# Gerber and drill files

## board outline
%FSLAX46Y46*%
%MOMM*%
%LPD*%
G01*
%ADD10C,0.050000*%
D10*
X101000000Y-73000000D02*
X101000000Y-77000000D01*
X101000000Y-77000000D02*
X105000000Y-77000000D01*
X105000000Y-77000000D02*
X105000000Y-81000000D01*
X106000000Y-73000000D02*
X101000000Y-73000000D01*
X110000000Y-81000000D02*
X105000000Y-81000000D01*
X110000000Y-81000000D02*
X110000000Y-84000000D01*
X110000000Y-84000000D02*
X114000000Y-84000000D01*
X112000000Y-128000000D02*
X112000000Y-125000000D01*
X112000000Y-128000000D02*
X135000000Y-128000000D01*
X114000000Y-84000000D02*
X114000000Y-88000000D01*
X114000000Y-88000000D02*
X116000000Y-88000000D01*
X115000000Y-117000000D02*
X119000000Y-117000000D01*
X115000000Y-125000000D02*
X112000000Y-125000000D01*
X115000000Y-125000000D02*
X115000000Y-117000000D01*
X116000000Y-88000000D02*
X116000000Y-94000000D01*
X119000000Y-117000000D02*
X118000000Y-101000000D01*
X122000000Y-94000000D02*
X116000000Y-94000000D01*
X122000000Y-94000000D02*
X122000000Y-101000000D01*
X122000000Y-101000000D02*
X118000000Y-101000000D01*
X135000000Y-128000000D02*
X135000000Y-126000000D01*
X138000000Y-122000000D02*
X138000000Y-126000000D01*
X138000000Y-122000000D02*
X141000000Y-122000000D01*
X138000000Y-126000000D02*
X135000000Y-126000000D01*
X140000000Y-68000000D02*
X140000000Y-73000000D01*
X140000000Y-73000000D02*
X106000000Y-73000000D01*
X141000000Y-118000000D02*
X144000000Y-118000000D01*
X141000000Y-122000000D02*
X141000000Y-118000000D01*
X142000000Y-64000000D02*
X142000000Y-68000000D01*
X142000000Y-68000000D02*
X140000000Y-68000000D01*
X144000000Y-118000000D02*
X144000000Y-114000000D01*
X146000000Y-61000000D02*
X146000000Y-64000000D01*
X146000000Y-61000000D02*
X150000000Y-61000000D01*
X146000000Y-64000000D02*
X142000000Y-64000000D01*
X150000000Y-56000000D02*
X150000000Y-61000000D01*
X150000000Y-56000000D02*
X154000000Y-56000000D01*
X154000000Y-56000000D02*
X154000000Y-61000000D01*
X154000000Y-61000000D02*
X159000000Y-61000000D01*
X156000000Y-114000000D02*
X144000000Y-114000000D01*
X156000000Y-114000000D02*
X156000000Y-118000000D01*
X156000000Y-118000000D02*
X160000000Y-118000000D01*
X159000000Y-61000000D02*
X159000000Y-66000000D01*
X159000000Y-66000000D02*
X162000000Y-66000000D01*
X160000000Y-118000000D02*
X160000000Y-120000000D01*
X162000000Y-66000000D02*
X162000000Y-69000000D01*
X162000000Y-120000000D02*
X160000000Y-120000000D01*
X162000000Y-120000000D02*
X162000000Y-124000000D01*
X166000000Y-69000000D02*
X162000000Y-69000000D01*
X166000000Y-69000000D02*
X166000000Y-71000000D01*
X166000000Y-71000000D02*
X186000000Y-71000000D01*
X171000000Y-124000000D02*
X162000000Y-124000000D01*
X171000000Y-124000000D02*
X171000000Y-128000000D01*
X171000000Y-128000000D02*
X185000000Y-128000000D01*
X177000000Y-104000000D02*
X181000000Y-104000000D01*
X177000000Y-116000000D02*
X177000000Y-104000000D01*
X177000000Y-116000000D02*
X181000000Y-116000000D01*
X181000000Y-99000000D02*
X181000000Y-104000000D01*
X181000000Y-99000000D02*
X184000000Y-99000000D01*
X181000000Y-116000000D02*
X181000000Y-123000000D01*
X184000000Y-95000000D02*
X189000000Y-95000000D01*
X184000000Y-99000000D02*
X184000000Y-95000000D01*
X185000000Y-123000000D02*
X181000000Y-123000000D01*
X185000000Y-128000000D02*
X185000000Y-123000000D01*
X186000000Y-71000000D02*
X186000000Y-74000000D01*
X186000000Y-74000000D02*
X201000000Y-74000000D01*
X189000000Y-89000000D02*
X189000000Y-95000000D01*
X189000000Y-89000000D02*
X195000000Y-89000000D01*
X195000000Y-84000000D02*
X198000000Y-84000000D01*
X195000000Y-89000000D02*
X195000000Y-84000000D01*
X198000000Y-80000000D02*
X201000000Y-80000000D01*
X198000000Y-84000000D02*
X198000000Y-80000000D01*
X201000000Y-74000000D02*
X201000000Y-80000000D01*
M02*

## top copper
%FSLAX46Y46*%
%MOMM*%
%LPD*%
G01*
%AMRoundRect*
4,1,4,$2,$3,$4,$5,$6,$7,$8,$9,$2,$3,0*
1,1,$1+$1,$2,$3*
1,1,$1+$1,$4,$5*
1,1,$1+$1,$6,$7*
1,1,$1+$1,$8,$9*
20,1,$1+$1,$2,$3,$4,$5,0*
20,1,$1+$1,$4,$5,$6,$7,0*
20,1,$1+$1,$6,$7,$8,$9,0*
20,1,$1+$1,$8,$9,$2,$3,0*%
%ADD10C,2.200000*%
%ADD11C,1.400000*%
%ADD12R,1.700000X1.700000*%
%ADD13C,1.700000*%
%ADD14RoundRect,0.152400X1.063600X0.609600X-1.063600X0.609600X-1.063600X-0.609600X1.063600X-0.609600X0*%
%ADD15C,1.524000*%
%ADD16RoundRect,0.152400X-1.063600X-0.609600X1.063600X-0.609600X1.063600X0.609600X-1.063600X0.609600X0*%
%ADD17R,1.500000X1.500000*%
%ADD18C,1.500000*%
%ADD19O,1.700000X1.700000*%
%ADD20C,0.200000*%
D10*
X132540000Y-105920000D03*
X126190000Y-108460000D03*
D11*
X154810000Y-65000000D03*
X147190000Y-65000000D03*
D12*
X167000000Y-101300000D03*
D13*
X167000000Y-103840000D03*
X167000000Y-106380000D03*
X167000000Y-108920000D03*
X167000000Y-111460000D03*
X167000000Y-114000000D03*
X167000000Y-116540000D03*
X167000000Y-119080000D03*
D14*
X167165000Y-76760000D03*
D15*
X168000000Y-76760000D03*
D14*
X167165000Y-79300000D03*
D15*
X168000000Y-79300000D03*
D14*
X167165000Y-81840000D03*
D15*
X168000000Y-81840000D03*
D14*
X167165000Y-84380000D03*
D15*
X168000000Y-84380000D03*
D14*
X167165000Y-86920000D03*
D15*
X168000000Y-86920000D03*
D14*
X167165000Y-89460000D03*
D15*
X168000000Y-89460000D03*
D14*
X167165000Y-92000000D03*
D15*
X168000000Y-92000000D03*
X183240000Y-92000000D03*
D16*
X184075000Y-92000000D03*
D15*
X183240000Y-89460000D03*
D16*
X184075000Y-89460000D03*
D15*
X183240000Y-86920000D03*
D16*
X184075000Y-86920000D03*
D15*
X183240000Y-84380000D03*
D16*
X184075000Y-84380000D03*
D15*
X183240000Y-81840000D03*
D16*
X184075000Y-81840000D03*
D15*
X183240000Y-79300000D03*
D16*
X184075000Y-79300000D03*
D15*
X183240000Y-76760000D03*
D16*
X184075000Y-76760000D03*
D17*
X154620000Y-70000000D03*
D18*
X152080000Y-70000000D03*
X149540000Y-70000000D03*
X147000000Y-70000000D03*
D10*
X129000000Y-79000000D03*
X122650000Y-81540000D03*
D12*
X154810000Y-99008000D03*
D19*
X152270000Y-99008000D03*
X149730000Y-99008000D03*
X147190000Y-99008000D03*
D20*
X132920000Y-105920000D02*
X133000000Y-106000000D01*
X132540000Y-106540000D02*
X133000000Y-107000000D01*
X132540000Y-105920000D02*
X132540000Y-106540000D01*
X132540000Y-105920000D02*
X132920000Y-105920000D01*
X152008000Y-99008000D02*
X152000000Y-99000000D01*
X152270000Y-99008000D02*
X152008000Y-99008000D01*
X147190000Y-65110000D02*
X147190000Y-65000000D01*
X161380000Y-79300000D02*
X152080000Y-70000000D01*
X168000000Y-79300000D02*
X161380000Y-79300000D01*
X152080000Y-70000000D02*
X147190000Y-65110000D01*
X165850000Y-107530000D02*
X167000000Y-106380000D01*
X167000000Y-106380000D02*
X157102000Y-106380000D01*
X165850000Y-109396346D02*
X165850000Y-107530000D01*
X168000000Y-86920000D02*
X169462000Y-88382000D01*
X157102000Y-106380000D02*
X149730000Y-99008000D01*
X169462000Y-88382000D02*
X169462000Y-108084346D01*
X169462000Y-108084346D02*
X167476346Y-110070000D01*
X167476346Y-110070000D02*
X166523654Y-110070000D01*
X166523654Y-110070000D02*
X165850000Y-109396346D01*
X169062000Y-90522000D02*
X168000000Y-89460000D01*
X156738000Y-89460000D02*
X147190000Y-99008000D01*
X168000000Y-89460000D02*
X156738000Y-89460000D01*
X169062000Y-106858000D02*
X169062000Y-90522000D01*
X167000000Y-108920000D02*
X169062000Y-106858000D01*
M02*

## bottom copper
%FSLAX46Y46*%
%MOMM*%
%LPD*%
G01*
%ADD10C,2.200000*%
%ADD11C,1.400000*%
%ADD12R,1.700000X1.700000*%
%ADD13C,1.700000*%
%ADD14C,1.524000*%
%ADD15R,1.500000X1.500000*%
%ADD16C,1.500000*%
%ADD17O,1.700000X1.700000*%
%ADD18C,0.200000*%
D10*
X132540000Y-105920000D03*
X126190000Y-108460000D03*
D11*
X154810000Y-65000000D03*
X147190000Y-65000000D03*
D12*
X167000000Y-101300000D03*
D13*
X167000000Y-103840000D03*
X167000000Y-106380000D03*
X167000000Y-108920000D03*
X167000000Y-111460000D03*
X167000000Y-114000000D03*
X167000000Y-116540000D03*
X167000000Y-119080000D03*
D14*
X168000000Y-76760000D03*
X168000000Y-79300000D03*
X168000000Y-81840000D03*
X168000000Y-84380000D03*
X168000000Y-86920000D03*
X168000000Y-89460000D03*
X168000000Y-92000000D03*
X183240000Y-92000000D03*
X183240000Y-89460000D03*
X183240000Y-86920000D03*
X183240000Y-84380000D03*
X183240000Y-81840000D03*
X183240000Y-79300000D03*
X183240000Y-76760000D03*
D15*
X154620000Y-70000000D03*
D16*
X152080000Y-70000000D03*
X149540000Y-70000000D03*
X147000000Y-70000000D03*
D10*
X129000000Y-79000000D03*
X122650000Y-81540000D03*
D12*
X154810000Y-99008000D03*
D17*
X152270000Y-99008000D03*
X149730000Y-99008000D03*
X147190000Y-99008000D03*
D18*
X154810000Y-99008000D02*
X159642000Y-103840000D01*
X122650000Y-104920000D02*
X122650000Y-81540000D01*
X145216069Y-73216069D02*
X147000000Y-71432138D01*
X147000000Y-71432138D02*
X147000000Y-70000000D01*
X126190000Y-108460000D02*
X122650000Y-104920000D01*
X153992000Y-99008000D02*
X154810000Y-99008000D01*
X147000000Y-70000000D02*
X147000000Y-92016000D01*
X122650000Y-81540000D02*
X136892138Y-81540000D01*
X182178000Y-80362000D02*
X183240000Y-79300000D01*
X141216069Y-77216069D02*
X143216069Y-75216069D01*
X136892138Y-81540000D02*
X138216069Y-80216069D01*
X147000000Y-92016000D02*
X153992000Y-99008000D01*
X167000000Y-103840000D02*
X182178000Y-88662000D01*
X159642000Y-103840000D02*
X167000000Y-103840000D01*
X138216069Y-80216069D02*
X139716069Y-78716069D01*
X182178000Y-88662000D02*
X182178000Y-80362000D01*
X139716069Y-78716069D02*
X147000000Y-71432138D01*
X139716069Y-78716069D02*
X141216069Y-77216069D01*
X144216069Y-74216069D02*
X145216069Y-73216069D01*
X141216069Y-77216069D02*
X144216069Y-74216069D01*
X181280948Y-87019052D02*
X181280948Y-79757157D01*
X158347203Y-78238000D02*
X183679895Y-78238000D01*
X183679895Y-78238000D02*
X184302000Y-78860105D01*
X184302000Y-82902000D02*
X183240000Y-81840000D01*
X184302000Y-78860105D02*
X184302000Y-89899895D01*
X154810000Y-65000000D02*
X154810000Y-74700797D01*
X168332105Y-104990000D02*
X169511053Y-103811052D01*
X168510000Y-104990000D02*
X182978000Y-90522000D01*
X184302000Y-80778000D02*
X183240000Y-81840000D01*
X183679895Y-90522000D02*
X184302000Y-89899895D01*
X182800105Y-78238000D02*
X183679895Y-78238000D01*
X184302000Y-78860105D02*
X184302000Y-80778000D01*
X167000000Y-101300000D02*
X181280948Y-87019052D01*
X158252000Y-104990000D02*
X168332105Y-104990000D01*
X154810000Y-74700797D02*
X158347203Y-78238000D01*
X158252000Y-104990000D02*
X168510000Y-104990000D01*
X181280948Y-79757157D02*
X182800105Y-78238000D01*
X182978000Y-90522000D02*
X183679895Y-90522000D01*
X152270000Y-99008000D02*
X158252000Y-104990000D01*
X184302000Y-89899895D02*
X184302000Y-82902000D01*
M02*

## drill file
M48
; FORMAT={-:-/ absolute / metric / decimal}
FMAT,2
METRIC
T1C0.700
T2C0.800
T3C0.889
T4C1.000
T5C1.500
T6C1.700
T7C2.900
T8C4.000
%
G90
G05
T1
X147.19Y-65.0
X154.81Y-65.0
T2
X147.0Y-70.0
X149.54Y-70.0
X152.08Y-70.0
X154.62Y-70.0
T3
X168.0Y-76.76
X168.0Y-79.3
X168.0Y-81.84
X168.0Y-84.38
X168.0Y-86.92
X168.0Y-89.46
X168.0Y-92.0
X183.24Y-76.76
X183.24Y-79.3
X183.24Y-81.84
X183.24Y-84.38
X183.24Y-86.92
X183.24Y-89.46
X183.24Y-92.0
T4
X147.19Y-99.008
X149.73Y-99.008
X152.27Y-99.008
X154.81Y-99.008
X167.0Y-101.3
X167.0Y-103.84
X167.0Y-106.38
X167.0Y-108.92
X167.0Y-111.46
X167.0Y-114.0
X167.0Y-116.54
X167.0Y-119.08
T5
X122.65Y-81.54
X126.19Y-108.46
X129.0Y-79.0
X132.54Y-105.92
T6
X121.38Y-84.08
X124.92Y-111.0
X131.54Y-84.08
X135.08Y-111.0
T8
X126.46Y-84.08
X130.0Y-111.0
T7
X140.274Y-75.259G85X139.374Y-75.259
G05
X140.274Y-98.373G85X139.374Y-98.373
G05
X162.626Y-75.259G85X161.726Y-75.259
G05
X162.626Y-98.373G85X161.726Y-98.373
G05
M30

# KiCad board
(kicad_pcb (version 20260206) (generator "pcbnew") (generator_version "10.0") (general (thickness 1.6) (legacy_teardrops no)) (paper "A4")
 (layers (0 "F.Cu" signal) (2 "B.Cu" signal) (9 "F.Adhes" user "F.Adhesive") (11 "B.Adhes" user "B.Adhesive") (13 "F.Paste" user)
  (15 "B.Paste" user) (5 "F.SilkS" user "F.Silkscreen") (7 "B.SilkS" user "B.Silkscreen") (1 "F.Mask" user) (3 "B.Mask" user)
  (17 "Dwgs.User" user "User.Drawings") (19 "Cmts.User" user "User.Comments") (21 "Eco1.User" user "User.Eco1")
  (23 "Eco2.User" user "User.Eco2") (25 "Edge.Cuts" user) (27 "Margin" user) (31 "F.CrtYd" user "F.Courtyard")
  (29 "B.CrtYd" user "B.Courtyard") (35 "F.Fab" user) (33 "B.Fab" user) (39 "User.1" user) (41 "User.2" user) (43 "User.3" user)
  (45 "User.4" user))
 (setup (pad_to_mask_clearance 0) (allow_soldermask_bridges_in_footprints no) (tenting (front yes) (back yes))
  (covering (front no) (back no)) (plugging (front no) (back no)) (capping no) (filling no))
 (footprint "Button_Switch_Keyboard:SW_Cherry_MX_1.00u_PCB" (layer "F.Cu") (at 132.54 105.92)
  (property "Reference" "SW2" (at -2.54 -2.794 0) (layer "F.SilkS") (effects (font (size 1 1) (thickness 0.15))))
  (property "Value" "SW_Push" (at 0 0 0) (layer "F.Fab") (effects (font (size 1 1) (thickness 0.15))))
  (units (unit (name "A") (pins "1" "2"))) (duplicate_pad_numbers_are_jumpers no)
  (pad "" np_thru_hole circle (at -7.62 5.08) (size 1.7 1.7) (drill 1.7) (layers "*.Cu" "*.Mask"))
  (pad "" np_thru_hole circle (at -2.54 5.08) (size 4 4) (drill 4) (layers "*.Cu" "*.Mask"))
  (pad "" np_thru_hole circle (at 2.54 5.08) (size 1.7 1.7) (drill 1.7) (layers "*.Cu" "*.Mask"))
  (pad "1" thru_hole circle (at 0 0) (size 2.2 2.2) (drill 1.5) (layers "*.Cu" "*.Mask") (remove_unused_layers no) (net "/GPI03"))
  (pad "2" thru_hole circle (at -6.35 2.54) (size 2.2 2.2) (drill 1.5) (layers "*.Cu" "*.Mask") (remove_unused_layers no) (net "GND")))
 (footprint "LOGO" (layer "F.Cu") (at 160 112)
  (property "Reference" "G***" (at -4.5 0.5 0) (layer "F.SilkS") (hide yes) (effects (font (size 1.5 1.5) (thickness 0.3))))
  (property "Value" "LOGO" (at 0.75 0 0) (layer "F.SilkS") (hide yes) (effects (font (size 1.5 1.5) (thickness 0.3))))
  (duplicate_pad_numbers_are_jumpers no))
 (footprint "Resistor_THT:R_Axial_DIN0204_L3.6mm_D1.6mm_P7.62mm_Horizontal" (layer "F.Cu") (at 154.81 65 180)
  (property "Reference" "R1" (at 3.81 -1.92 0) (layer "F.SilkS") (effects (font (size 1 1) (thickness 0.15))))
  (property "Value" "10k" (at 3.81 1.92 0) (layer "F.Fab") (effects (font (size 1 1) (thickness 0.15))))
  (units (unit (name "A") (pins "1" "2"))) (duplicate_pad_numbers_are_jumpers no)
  (pad "1" thru_hole circle (at 0 0 180) (size 1.4 1.4) (drill 0.7) (layers "*.Cu" "*.Mask") (remove_unused_layers no) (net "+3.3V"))
  (pad "2" thru_hole circle (at 7.62 0 180) (size 1.4 1.4) (drill 0.7) (layers "*.Cu" "*.Mask") (remove_unused_layers no)
   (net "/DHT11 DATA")))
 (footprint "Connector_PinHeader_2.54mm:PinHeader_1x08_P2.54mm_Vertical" (layer "F.Cu") (at 167 101.3)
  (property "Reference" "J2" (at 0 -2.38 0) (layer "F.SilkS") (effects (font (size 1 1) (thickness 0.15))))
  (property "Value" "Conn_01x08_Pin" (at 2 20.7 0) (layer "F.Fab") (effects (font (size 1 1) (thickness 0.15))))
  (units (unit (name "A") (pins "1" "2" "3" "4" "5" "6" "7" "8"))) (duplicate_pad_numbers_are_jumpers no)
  (pad "1" thru_hole rect (at 0 0) (size 1.7 1.7) (drill 1) (layers "*.Cu" "*.Mask") (remove_unused_layers no) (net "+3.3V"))
  (pad "2" thru_hole circle (at 0 2.54) (size 1.7 1.7) (drill 1) (layers "*.Cu" "*.Mask") (remove_unused_layers no) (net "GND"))
  (pad "3" thru_hole circle (at 0 5.08) (size 1.7 1.7) (drill 1) (layers "*.Cu" "*.Mask") (remove_unused_layers no) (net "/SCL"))
  (pad "4" thru_hole circle (at 0 7.62) (size 1.7 1.7) (drill 1) (layers "*.Cu" "*.Mask") (remove_unused_layers no) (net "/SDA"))
  (pad "5" thru_hole circle (at 0 10.16) (size 1.7 1.7) (drill 1) (layers "*.Cu" "*.Mask") (remove_unused_layers no)
   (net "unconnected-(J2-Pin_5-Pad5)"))
  (pad "6" thru_hole circle (at 0 12.7) (size 1.7 1.7) (drill 1) (layers "*.Cu" "*.Mask") (remove_unused_layers no)
   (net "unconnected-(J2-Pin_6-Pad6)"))
  (pad "7" thru_hole circle (at 0 15.24) (size 1.7 1.7) (drill 1) (layers "*.Cu" "*.Mask") (remove_unused_layers no)
   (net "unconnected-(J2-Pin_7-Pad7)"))
  (pad "8" thru_hole circle (at 0 17.78) (size 1.7 1.7) (drill 1) (layers "*.Cu" "*.Mask") (remove_unused_layers no)
   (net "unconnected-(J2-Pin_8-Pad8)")))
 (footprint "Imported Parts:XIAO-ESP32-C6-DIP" (layer "F.Cu") (at 175.62 84.38 90)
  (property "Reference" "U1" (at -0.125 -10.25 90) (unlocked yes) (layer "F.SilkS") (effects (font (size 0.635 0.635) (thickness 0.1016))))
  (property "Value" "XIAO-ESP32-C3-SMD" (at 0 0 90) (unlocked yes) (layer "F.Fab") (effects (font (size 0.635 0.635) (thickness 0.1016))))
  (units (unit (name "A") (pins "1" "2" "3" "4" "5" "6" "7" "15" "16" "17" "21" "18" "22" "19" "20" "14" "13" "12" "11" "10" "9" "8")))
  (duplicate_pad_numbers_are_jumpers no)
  (pad "1" smd roundrect (at 7.62 -8.455 180) (size 2.432 1.524) (layers "F.Cu" "F.Mask") (roundrect_rratio 0.1)
   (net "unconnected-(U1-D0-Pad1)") (thermal_bridge_angle 45))
  (pad "1" thru_hole circle (at 7.62 -7.62 180) (size 1.524 1.524) (drill 0.889) (layers "*.Cu" "*.Mask") (remove_unused_layers no)
   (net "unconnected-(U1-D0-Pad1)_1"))
  (pad "2" smd roundrect (at 5.08 -8.455 180) (size 2.432 1.524) (layers "F.Cu" "F.Mask") (roundrect_rratio 0.1) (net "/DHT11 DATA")
   (thermal_bridge_angle 45))
  (pad "2" thru_hole circle (at 5.08 -7.62 180) (size 1.524 1.524) (drill 0.889) (layers "*.Cu" "*.Mask") (remove_unused_layers no)
   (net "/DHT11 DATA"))
  (pad "3" smd roundrect (at 2.54 -8.455 180) (size 2.432 1.524) (layers "F.Cu" "F.Mask") (roundrect_rratio 0.1) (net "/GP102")
   (thermal_bridge_angle 45))
  (pad "3" thru_hole circle (at 2.54 -7.62 180) (size 1.524 1.524) (drill 0.889) (layers "*.Cu" "*.Mask") (remove_unused_layers no)
   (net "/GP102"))
  (pad "4" smd roundrect (at 0 -8.455 180) (size 2.432 1.524) (layers "F.Cu" "F.Mask") (roundrect_rratio 0.1) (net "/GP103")
   (thermal_bridge_angle 45))
  (pad "4" thru_hole circle (at 0 -7.62 180) (size 1.524 1.524) (drill 0.889) (layers "*.Cu" "*.Mask") (remove_unused_layers no)
   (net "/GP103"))
  (pad "5" smd roundrect (at -2.54 -8.455 180) (size 2.432 1.524) (layers "F.Cu" "F.Mask") (roundrect_rratio 0.1) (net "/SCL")
   (thermal_bridge_angle 45))
  (pad "5" thru_hole circle (at -2.54 -7.62 180) (size 1.524 1.524) (drill 0.889) (layers "*.Cu" "*.Mask") (remove_unused_layers no)
   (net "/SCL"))
  (pad "6" smd roundrect (at -5.08 -8.455 180) (size 2.432 1.524) (layers "F.Cu" "F.Mask") (roundrect_rratio 0.1) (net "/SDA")
   (thermal_bridge_angle 45))
  (pad "6" thru_hole circle (at -5.08 -7.62 180) (size 1.524 1.524) (drill 0.889) (layers "*.Cu" "*.Mask") (remove_unused_layers no)
   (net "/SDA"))
  (pad "7" smd roundrect (at -7.62 -8.455 180) (size 2.432 1.524) (layers "F.Cu" "F.Mask") (roundrect_rratio 0.1)
   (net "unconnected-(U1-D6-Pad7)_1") (thermal_bridge_angle 45))
  (pad "7" thru_hole circle (at -7.62 -7.62 180) (size 1.524 1.524) (drill 0.889) (layers "*.Cu" "*.Mask") (remove_unused_layers no)
   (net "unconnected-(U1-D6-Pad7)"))
  (pad "8" thru_hole circle (at -7.62 7.62) (size 1.524 1.524) (drill 0.889) (layers "*.Cu" "*.Mask") (remove_unused_layers no)
   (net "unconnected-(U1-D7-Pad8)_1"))
  (pad "8" smd roundrect (at -7.62 8.455) (size 2.432 1.524) (layers "F.Cu" "F.Mask") (roundrect_rratio 0.1)
   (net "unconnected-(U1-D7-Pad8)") (thermal_bridge_angle 45))
  (pad "9" thru_hole circle (at -5.08 7.62) (size 1.524 1.524) (drill 0.889) (layers "*.Cu" "*.Mask") (remove_unused_layers no)
   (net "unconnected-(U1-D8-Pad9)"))
  (pad "9" smd roundrect (at -5.08 8.455) (size 2.432 1.524) (layers "F.Cu" "F.Mask") (roundrect_rratio 0.1)
   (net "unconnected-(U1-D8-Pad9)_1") (thermal_bridge_angle 45))
  (pad "10" thru_hole circle (at -2.54 7.62) (size 1.524 1.524) (drill 0.889) (layers "*.Cu" "*.Mask") (remove_unused_layers no)
   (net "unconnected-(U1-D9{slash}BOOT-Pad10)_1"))
  (pad "10" smd roundrect (at -2.54 8.455) (size 2.432 1.524) (layers "F.Cu" "F.Mask") (roundrect_rratio 0.1)
   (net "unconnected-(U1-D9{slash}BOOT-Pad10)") (thermal_bridge_angle 45))
  (pad "11" thru_hole circle (at 0 7.62) (size 1.524 1.524) (drill 0.889) (layers "*.Cu" "*.Mask") (remove_unused_layers no)
   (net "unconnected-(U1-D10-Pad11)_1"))
  (pad "11" smd roundrect (at 0 8.455) (size 2.432 1.524) (layers "F.Cu" "F.Mask") (roundrect_rratio 0.1) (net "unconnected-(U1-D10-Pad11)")
   (thermal_bridge_angle 45))
  (pad "12" thru_hole circle (at 2.54 7.62) (size 1.524 1.524) (drill 0.889) (layers "*.Cu" "*.Mask") (remove_unused_layers no)
   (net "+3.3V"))
  (pad "12" smd roundrect (at 2.54 8.455) (size 2.432 1.524) (layers "F.Cu" "F.Mask") (roundrect_rratio 0.1) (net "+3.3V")
   (thermal_bridge_angle 45))
  (pad "13" thru_hole circle (at 5.08 7.62) (size 1.524 1.524) (drill 0.889) (layers "*.Cu" "*.Mask") (remove_unused_layers no) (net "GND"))
  (pad "13" smd roundrect (at 5.08 8.455) (size 2.432 1.524) (layers "F.Cu" "F.Mask") (roundrect_rratio 0.1) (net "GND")
   (thermal_bridge_angle 45))
  (pad "14" thru_hole circle (at 7.62 7.62) (size 1.524 1.524) (drill 0.889) (layers "*.Cu" "*.Mask") (remove_unused_layers no) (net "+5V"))
  (pad "14" smd roundrect (at 7.62 8.455) (size 2.432 1.524) (layers "F.Cu" "F.Mask") (roundrect_rratio 0.1) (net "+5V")
   (thermal_bridge_angle 45)))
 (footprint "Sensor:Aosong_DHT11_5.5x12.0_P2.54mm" (layer "F.Cu") (at 154.62 70 -90)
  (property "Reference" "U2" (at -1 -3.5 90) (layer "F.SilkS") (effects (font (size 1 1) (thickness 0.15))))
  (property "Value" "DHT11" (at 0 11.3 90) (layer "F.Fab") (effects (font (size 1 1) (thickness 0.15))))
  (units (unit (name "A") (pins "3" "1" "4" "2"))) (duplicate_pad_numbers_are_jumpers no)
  (pad "1" thru_hole rect (at 0 0 270) (size 1.5 1.5) (drill 0.8) (layers "*.Cu" "*.Mask") (remove_unused_layers no) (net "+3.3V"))
  (pad "2" thru_hole circle (at 0 2.54 270) (size 1.5 1.5) (drill 0.8) (layers "*.Cu" "*.Mask") (remove_unused_layers no)
   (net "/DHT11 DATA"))
  (pad "3" thru_hole circle (at 0 5.08 270) (size 1.5 1.5) (drill 0.8) (layers "*.Cu" "*.Mask") (remove_unused_layers no)
   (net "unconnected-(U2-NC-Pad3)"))
  (pad "4" thru_hole circle (at 0 7.62 270) (size 1.5 1.5) (drill 0.8) (layers "*.Cu" "*.Mask") (remove_unused_layers no) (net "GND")))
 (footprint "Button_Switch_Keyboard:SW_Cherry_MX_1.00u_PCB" (layer "F.Cu") (at 129 79)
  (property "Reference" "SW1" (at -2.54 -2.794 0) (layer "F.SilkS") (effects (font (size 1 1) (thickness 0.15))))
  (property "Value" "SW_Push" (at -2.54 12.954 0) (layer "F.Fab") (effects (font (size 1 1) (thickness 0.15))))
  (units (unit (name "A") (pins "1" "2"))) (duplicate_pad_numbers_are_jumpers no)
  (pad "" np_thru_hole circle (at -7.62 5.08) (size 1.7 1.7) (drill 1.7) (layers "*.Cu" "*.Mask"))
  (pad "" np_thru_hole circle (at -2.54 5.08) (size 4 4) (drill 4) (layers "*.Cu" "*.Mask"))
  (pad "" np_thru_hole circle (at 2.54 5.08) (size 1.7 1.7) (drill 1.7) (layers "*.Cu" "*.Mask"))
  (pad "1" thru_hole circle (at 0 0) (size 2.2 2.2) (drill 1.5) (layers "*.Cu" "*.Mask") (remove_unused_layers no) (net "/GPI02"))
  (pad "2" thru_hole circle (at -6.35 2.54) (size 2.2 2.2) (drill 1.5) (layers "*.Cu" "*.Mask") (remove_unused_layers no) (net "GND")))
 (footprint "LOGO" (layer "F.Cu") (at 191.5 80.5)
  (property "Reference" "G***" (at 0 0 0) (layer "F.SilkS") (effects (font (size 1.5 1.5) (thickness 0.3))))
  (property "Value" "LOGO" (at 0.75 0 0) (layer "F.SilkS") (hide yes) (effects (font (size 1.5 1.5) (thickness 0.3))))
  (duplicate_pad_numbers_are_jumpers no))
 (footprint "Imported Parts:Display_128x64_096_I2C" (layer "F.Cu") (at 151 99.008 180)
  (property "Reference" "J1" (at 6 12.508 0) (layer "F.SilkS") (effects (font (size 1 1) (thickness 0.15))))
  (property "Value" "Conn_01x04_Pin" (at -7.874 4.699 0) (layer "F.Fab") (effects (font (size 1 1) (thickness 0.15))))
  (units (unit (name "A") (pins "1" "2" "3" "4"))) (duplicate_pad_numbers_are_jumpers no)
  (pad "" np_thru_hole oval (at -11.176 0.635 180) (size 3.8 2.9) (drill oval 3.8 2.9) (layers "*.Cu" "*.Mask"))
  (pad "" np_thru_hole oval (at -11.176 23.749 180) (size 3.8 2.9) (drill oval 3.8 2.9) (layers "*.Cu" "*.Mask"))
  (pad "" np_thru_hole oval (at 11.176 0.635 180) (size 3.8 2.9) (drill oval 3.8 2.9) (layers "*.Cu" "*.Mask"))
  (pad "" np_thru_hole oval (at 11.176 23.749 180) (size 3.8 2.9) (drill oval 3.8 2.9) (layers "*.Cu" "*.Mask"))
  (pad "1" thru_hole rect (at -3.81 0 270) (size 1.7 1.7) (drill 1) (layers "*.Cu" "*.Mask") (remove_unused_layers no) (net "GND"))
  (pad "2" thru_hole oval (at -1.27 0 270) (size 1.7 1.7) (drill 1) (layers "*.Cu" "*.Mask") (remove_unused_layers no) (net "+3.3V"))
  (pad "3" thru_hole oval (at 1.27 0 270) (size 1.7 1.7) (drill 1) (layers "*.Cu" "*.Mask") (remove_unused_layers no) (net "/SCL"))
  (pad "4" thru_hole oval (at 3.81 0 270) (size 1.7 1.7) (drill 1) (layers "*.Cu" "*.Mask") (remove_unused_layers no) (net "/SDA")))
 (gr_line (start 101 73) (end 101 77) (stroke (width 0.05) (type default)) (layer "Edge.Cuts"))
 (gr_line (start 101 77) (end 105 77) (stroke (width 0.05) (type default)) (layer "Edge.Cuts"))
 (gr_line (start 105 77) (end 105 81) (stroke (width 0.05) (type default)) (layer "Edge.Cuts"))
 (gr_line (start 106 73) (end 101 73) (stroke (width 0.05) (type default)) (layer "Edge.Cuts"))
 (gr_line (start 110 81) (end 105 81) (stroke (width 0.05) (type default)) (layer "Edge.Cuts"))
 (gr_line (start 110 81) (end 110 84) (stroke (width 0.05) (type default)) (layer "Edge.Cuts"))
 (gr_line (start 110 84) (end 114 84) (stroke (width 0.05) (type default)) (layer "Edge.Cuts"))
 (gr_line (start 112 128) (end 112 125) (stroke (width 0.05) (type default)) (layer "Edge.Cuts"))
 (gr_line (start 112 128) (end 135 128) (stroke (width 0.05) (type default)) (layer "Edge.Cuts"))
 (gr_line (start 114 84) (end 114 88) (stroke (width 0.05) (type default)) (layer "Edge.Cuts"))
 (gr_line (start 114 88) (end 116 88) (stroke (width 0.05) (type default)) (layer "Edge.Cuts"))
 (gr_line (start 115 117) (end 119 117) (stroke (width 0.05) (type default)) (layer "Edge.Cuts"))
 (gr_line (start 115 125) (end 112 125) (stroke (width 0.05) (type default)) (layer "Edge.Cuts"))
 (gr_line (start 115 125) (end 115 117) (stroke (width 0.05) (type default)) (layer "Edge.Cuts"))
 (gr_line (start 116 88) (end 116 94) (stroke (width 0.05) (type default)) (layer "Edge.Cuts"))
 (gr_line (start 119 117) (end 118 101) (stroke (width 0.05) (type default)) (layer "Edge.Cuts"))
 (gr_line (start 122 94) (end 116 94) (stroke (width 0.05) (type default)) (layer "Edge.Cuts"))
 (gr_line (start 122 94) (end 122 101) (stroke (width 0.05) (type default)) (layer "Edge.Cuts"))
 (gr_line (start 122 101) (end 118 101) (stroke (width 0.05) (type default)) (layer "Edge.Cuts"))
 (gr_line (start 135 128) (end 135 126) (stroke (width 0.05) (type default)) (layer "Edge.Cuts"))
 (gr_line (start 138 122) (end 138 126) (stroke (width 0.05) (type default)) (layer "Edge.Cuts"))
 (gr_line (start 138 122) (end 141 122) (stroke (width 0.05) (type default)) (layer "Edge.Cuts"))
 (gr_line (start 138 126) (end 135 126) (stroke (width 0.05) (type default)) (layer "Edge.Cuts"))
 (gr_line (start 140 68) (end 140 73) (stroke (width 0.05) (type default)) (layer "Edge.Cuts"))
 (gr_line (start 140 73) (end 106 73) (stroke (width 0.05) (type default)) (layer "Edge.Cuts"))
 (gr_line (start 141 118) (end 144 118) (stroke (width 0.05) (type default)) (layer "Edge.Cuts"))
 (gr_line (start 141 122) (end 141 118) (stroke (width 0.05) (type default)) (layer "Edge.Cuts"))
 (gr_line (start 142 64) (end 142 68) (stroke (width 0.05) (type default)) (layer "Edge.Cuts"))
 (gr_line (start 142 68) (end 140 68) (stroke (width 0.05) (type default)) (layer "Edge.Cuts"))
 (gr_line (start 144 118) (end 144 114) (stroke (width 0.05) (type default)) (layer "Edge.Cuts"))
 (gr_line (start 146 61) (end 146 64) (stroke (width 0.05) (type default)) (layer "Edge.Cuts"))
 (gr_line (start 146 61) (end 150 61) (stroke (width 0.05) (type default)) (layer "Edge.Cuts"))
 (gr_line (start 146 64) (end 142 64) (stroke (width 0.05) (type default)) (layer "Edge.Cuts"))
 (gr_line (start 150 56) (end 150 61) (stroke (width 0.05) (type default)) (layer "Edge.Cuts"))
 (gr_line (start 150 56) (end 154 56) (stroke (width 0.05) (type default)) (layer "Edge.Cuts"))
 (gr_line (start 154 56) (end 154 61) (stroke (width 0.05) (type default)) (layer "Edge.Cuts"))
 (gr_line (start 154 61) (end 159 61) (stroke (width 0.05) (type default)) (layer "Edge.Cuts"))
 (gr_line (start 156 114) (end 144 114) (stroke (width 0.05) (type default)) (layer "Edge.Cuts"))
 (gr_line (start 156 114) (end 156 118) (stroke (width 0.05) (type default)) (layer "Edge.Cuts"))
 (gr_line (start 156 118) (end 160 118) (stroke (width 0.05) (type default)) (layer "Edge.Cuts"))
 (gr_line (start 159 61) (end 159 66) (stroke (width 0.05) (type default)) (layer "Edge.Cuts"))
 (gr_line (start 159 66) (end 162 66) (stroke (width 0.05) (type default)) (layer "Edge.Cuts"))
 (gr_line (start 160 118) (end 160 120) (stroke (width 0.05) (type default)) (layer "Edge.Cuts"))
 (gr_line (start 162 66) (end 162 69) (stroke (width 0.05) (type default)) (layer "Edge.Cuts"))
 (gr_line (start 162 120) (end 160 120) (stroke (width 0.05) (type default)) (layer "Edge.Cuts"))
 (gr_line (start 162 120) (end 162 124) (stroke (width 0.05) (type default)) (layer "Edge.Cuts"))
 (gr_line (start 166 69) (end 162 69) (stroke (width 0.05) (type default)) (layer "Edge.Cuts"))
 (gr_line (start 166 69) (end 166 71) (stroke (width 0.05) (type default)) (layer "Edge.Cuts"))
 (gr_line (start 166 71) (end 186 71) (stroke (width 0.05) (type default)) (layer "Edge.Cuts"))
 (gr_line (start 171 124) (end 162 124) (stroke (width 0.05) (type default)) (layer "Edge.Cuts"))
 (gr_line (start 171 124) (end 171 128) (stroke (width 0.05) (type default)) (layer "Edge.Cuts"))
 (gr_line (start 171 128) (end 185 128) (stroke (width 0.05) (type default)) (layer "Edge.Cuts"))
 (gr_line (start 177 104) (end 181 104) (stroke (width 0.05) (type default)) (layer "Edge.Cuts"))
 (gr_line (start 177 116) (end 177 104) (stroke (width 0.05) (type default)) (layer "Edge.Cuts"))
 (gr_line (start 177 116) (end 181 116) (stroke (width 0.05) (type default)) (layer "Edge.Cuts"))
 (gr_line (start 181 99) (end 181 104) (stroke (width 0.05) (type default)) (layer "Edge.Cuts"))
 (gr_line (start 181 99) (end 184 99) (stroke (width 0.05) (type default)) (layer "Edge.Cuts"))
 (gr_line (start 181 116) (end 181 123) (stroke (width 0.05) (type default)) (layer "Edge.Cuts"))
 (gr_line (start 184 95) (end 189 95) (stroke (width 0.05) (type default)) (layer "Edge.Cuts"))
 (gr_line (start 184 99) (end 184 95) (stroke (width 0.05) (type default)) (layer "Edge.Cuts"))
 (gr_line (start 185 123) (end 181 123) (stroke (width 0.05) (type default)) (layer "Edge.Cuts"))
 (gr_line (start 185 128) (end 185 123) (stroke (width 0.05) (type default)) (layer "Edge.Cuts"))
 (gr_line (start 186 71) (end 186 74) (stroke (width 0.05) (type default)) (layer "Edge.Cuts"))
 (gr_line (start 186 74) (end 201 74) (stroke (width 0.05) (type default)) (layer "Edge.Cuts"))
 (gr_line (start 189 89) (end 189 95) (stroke (width 0.05) (type default)) (layer "Edge.Cuts"))
 (gr_line (start 189 89) (end 195 89) (stroke (width 0.05) (type default)) (layer "Edge.Cuts"))
 (gr_line (start 195 84) (end 198 84) (stroke (width 0.05) (type default)) (layer "Edge.Cuts"))
 (gr_line (start 195 89) (end 195 84) (stroke (width 0.05) (type default)) (layer "Edge.Cuts"))
 (gr_line (start 198 80) (end 201 80) (stroke (width 0.05) (type default)) (layer "Edge.Cuts"))
 (gr_line (start 198 84) (end 198 80) (stroke (width 0.05) (type default)) (layer "Edge.Cuts"))
 (gr_line (start 201 74) (end 201 80) (stroke (width 0.05) (type default)) (layer "Edge.Cuts"))
 (segment (start 132.92 105.92) (end 133 106) (width 0.2) (layer "F.Cu") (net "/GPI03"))
 (segment (start 132.54 106.54) (end 133 107) (width 0.2) (layer "F.Cu") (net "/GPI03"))
 (segment (start 132.54 105.92) (end 132.54 106.54) (width 0.2) (layer "F.Cu") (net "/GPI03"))
 (segment (start 132.54 105.92) (end 132.92 105.92) (width 0.2) (layer "F.Cu") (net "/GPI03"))
 (segment (start 154.81 99.008) (end 159.642 103.84) (width 0.2) (layer "B.Cu") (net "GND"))
 (segment (start 122.65 104.92) (end 122.65 81.54) (width 0.2) (layer "B.Cu") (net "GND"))
 (segment (start 145.216069 73.216069) (end 147 71.432138) (width 0.2) (layer "B.Cu") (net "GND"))
 (segment (start 147 71.432138) (end 147 70) (width 0.2) (layer "B.Cu") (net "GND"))
 (segment (start 126.19 108.46) (end 122.65 104.92) (width 0.2) (layer "B.Cu") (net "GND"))
 (segment (start 153.992 99.008) (end 154.81 99.008) (width 0.2) (layer "B.Cu") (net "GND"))
 (segment (start 147 70) (end 147 92.016) (width 0.2) (layer "B.Cu") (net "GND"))
 (segment (start 122.65 81.54) (end 136.892138 81.54) (width 0.2) (layer "B.Cu") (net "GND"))
 (segment (start 182.178 80.362) (end 183.24 79.3) (width 0.2) (layer "B.Cu") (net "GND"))
 (segment (start 141.216069 77.216069) (end 143.216069 75.216069) (width 0.2) (layer "B.Cu") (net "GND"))
 (segment (start 136.892138 81.54) (end 138.216069 80.216069) (width 0.2) (layer "B.Cu") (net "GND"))
 (segment (start 147 92.016) (end 153.992 99.008) (width 0.2) (layer "B.Cu") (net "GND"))
 (segment (start 167 103.84) (end 182.178 88.662) (width 0.2) (layer "B.Cu") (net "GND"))
 (segment (start 159.642 103.84) (end 167 103.84) (width 0.2) (layer "B.Cu") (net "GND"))
 (segment (start 138.216069 80.216069) (end 139.716069 78.716069) (width 0.2) (layer "B.Cu") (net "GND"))
 (segment (start 182.178 88.662) (end 182.178 80.362) (width 0.2) (layer "B.Cu") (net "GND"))
 (segment (start 139.716069 78.716069) (end 147 71.432138) (width 0.2) (layer "B.Cu") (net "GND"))
 (segment (start 139.716069 78.716069) (end 141.216069 77.216069) (width 0.2) (layer "B.Cu") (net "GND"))
 (segment (start 144.216069 74.216069) (end 145.216069 73.216069) (width 0.2) (layer "B.Cu") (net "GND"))
 (segment (start 141.216069 77.216069) (end 144.216069 74.216069) (width 0.2) (layer "B.Cu") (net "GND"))
 (segment (start 152.008 99.008) (end 152 99) (width 0.2) (layer "F.Cu") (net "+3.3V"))
 (segment (start 152.27 99.008) (end 152.008 99.008) (width 0.2) (layer "F.Cu") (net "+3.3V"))
 (segment (start 181.280948 87.019052) (end 181.280948 79.757157) (width 0.2) (layer "B.Cu") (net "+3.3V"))
 (segment (start 158.347203 78.238) (end 183.679895 78.238) (width 0.2) (layer "B.Cu") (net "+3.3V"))
 (segment (start 183.679895 78.238) (end 184.302 78.860105) (width 0.2) (layer "B.Cu") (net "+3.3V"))
 (segment (start 184.302 82.902) (end 183.24 81.84) (width 0.2) (layer "B.Cu") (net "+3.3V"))
 (segment (start 184.302 78.860105) (end 184.302 89.899895) (width 0.2) (layer "B.Cu") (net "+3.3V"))
 (segment (start 154.81 65) (end 154.81 74.700797) (width 0.2) (layer "B.Cu") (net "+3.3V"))
 (segment (start 168.332105 104.99) (end 169.511053 103.811052) (width 0.2) (layer "B.Cu") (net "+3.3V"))
 (segment (start 168.51 104.99) (end 182.978 90.522) (width 0.2) (layer "B.Cu") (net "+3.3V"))
 (segment (start 184.302 80.778) (end 183.24 81.84) (width 0.2) (layer "B.Cu") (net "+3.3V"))
 (segment (start 183.679895 90.522) (end 184.302 89.899895) (width 0.2) (layer "B.Cu") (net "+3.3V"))
 (segment (start 182.800105 78.238) (end 183.679895 78.238) (width 0.2) (layer "B.Cu") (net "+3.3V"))
 (segment (start 184.302 78.860105) (end 184.302 80.778) (width 0.2) (layer "B.Cu") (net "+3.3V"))
 (segment (start 167 101.3) (end 181.280948 87.019052) (width 0.2) (layer "B.Cu") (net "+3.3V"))
 (segment (start 158.252 104.99) (end 168.332105 104.99) (width 0.2) (layer "B.Cu") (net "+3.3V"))
 (segment (start 154.81 74.700797) (end 158.347203 78.238) (width 0.2) (layer "B.Cu") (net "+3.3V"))
 (segment (start 158.252 104.99) (end 168.51 104.99) (width 0.2) (layer "B.Cu") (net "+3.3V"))
 (segment (start 181.280948 79.757157) (end 182.800105 78.238) (width 0.2) (layer "B.Cu") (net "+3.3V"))
 (segment (start 182.978 90.522) (end 183.679895 90.522) (width 0.2) (layer "B.Cu") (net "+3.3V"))
 (segment (start 152.27 99.008) (end 158.252 104.99) (width 0.2) (layer "B.Cu") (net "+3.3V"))
 (segment (start 184.302 89.899895) (end 184.302 82.902) (width 0.2) (layer "B.Cu") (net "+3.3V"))
 (segment (start 147.19 65.11) (end 147.19 65) (width 0.2) (layer "F.Cu") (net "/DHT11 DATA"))
 (segment (start 161.38 79.3) (end 152.08 70) (width 0.2) (layer "F.Cu") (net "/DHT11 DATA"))
 (segment (start 168 79.3) (end 161.38 79.3) (width 0.2) (layer "F.Cu") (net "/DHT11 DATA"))
 (segment (start 152.08 70) (end 147.19 65.11) (width 0.2) (layer "F.Cu") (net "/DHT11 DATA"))
 (segment (start 165.85 107.53) (end 167 106.38) (width 0.2) (layer "F.Cu") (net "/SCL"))
 (segment (start 167 106.38) (end 157.102 106.38) (width 0.2) (layer "F.Cu") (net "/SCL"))
 (segment (start 165.85 109.396346) (end 165.85 107.53) (width 0.2) (layer "F.Cu") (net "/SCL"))
 (segment (start 168 86.92) (end 169.462 88.382) (width 0.2) (layer "F.Cu") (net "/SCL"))
 (segment (start 157.102 106.38) (end 149.73 99.008) (width 0.2) (layer "F.Cu") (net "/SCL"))
 (segment (start 169.462 88.382) (end 169.462 108.084346) (width 0.2) (layer "F.Cu") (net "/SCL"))
 (segment (start 169.462 108.084346) (end 167.476346 110.07) (width 0.2) (layer "F.Cu") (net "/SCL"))
 (segment (start 167.476346 110.07) (end 166.523654 110.07) (width 0.2) (layer "F.Cu") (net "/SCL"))
 (segment (start 166.523654 110.07) (end 165.85 109.396346) (width 0.2) (layer "F.Cu") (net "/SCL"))
 (segment (start 169.062 90.522) (end 168 89.46) (width 0.2) (layer "F.Cu") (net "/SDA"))
 (segment (start 156.738 89.46) (end 147.19 99.008) (width 0.2) (layer "F.Cu") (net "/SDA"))
 (segment (start 168 89.46) (end 156.738 89.46) (width 0.2) (layer "F.Cu") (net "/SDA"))
 (segment (start 169.062 106.858) (end 169.062 90.522) (width 0.2) (layer "F.Cu") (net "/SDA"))
 (segment (start 167 108.92) (end 169.062 106.858) (width 0.2) (layer "F.Cu") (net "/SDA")))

